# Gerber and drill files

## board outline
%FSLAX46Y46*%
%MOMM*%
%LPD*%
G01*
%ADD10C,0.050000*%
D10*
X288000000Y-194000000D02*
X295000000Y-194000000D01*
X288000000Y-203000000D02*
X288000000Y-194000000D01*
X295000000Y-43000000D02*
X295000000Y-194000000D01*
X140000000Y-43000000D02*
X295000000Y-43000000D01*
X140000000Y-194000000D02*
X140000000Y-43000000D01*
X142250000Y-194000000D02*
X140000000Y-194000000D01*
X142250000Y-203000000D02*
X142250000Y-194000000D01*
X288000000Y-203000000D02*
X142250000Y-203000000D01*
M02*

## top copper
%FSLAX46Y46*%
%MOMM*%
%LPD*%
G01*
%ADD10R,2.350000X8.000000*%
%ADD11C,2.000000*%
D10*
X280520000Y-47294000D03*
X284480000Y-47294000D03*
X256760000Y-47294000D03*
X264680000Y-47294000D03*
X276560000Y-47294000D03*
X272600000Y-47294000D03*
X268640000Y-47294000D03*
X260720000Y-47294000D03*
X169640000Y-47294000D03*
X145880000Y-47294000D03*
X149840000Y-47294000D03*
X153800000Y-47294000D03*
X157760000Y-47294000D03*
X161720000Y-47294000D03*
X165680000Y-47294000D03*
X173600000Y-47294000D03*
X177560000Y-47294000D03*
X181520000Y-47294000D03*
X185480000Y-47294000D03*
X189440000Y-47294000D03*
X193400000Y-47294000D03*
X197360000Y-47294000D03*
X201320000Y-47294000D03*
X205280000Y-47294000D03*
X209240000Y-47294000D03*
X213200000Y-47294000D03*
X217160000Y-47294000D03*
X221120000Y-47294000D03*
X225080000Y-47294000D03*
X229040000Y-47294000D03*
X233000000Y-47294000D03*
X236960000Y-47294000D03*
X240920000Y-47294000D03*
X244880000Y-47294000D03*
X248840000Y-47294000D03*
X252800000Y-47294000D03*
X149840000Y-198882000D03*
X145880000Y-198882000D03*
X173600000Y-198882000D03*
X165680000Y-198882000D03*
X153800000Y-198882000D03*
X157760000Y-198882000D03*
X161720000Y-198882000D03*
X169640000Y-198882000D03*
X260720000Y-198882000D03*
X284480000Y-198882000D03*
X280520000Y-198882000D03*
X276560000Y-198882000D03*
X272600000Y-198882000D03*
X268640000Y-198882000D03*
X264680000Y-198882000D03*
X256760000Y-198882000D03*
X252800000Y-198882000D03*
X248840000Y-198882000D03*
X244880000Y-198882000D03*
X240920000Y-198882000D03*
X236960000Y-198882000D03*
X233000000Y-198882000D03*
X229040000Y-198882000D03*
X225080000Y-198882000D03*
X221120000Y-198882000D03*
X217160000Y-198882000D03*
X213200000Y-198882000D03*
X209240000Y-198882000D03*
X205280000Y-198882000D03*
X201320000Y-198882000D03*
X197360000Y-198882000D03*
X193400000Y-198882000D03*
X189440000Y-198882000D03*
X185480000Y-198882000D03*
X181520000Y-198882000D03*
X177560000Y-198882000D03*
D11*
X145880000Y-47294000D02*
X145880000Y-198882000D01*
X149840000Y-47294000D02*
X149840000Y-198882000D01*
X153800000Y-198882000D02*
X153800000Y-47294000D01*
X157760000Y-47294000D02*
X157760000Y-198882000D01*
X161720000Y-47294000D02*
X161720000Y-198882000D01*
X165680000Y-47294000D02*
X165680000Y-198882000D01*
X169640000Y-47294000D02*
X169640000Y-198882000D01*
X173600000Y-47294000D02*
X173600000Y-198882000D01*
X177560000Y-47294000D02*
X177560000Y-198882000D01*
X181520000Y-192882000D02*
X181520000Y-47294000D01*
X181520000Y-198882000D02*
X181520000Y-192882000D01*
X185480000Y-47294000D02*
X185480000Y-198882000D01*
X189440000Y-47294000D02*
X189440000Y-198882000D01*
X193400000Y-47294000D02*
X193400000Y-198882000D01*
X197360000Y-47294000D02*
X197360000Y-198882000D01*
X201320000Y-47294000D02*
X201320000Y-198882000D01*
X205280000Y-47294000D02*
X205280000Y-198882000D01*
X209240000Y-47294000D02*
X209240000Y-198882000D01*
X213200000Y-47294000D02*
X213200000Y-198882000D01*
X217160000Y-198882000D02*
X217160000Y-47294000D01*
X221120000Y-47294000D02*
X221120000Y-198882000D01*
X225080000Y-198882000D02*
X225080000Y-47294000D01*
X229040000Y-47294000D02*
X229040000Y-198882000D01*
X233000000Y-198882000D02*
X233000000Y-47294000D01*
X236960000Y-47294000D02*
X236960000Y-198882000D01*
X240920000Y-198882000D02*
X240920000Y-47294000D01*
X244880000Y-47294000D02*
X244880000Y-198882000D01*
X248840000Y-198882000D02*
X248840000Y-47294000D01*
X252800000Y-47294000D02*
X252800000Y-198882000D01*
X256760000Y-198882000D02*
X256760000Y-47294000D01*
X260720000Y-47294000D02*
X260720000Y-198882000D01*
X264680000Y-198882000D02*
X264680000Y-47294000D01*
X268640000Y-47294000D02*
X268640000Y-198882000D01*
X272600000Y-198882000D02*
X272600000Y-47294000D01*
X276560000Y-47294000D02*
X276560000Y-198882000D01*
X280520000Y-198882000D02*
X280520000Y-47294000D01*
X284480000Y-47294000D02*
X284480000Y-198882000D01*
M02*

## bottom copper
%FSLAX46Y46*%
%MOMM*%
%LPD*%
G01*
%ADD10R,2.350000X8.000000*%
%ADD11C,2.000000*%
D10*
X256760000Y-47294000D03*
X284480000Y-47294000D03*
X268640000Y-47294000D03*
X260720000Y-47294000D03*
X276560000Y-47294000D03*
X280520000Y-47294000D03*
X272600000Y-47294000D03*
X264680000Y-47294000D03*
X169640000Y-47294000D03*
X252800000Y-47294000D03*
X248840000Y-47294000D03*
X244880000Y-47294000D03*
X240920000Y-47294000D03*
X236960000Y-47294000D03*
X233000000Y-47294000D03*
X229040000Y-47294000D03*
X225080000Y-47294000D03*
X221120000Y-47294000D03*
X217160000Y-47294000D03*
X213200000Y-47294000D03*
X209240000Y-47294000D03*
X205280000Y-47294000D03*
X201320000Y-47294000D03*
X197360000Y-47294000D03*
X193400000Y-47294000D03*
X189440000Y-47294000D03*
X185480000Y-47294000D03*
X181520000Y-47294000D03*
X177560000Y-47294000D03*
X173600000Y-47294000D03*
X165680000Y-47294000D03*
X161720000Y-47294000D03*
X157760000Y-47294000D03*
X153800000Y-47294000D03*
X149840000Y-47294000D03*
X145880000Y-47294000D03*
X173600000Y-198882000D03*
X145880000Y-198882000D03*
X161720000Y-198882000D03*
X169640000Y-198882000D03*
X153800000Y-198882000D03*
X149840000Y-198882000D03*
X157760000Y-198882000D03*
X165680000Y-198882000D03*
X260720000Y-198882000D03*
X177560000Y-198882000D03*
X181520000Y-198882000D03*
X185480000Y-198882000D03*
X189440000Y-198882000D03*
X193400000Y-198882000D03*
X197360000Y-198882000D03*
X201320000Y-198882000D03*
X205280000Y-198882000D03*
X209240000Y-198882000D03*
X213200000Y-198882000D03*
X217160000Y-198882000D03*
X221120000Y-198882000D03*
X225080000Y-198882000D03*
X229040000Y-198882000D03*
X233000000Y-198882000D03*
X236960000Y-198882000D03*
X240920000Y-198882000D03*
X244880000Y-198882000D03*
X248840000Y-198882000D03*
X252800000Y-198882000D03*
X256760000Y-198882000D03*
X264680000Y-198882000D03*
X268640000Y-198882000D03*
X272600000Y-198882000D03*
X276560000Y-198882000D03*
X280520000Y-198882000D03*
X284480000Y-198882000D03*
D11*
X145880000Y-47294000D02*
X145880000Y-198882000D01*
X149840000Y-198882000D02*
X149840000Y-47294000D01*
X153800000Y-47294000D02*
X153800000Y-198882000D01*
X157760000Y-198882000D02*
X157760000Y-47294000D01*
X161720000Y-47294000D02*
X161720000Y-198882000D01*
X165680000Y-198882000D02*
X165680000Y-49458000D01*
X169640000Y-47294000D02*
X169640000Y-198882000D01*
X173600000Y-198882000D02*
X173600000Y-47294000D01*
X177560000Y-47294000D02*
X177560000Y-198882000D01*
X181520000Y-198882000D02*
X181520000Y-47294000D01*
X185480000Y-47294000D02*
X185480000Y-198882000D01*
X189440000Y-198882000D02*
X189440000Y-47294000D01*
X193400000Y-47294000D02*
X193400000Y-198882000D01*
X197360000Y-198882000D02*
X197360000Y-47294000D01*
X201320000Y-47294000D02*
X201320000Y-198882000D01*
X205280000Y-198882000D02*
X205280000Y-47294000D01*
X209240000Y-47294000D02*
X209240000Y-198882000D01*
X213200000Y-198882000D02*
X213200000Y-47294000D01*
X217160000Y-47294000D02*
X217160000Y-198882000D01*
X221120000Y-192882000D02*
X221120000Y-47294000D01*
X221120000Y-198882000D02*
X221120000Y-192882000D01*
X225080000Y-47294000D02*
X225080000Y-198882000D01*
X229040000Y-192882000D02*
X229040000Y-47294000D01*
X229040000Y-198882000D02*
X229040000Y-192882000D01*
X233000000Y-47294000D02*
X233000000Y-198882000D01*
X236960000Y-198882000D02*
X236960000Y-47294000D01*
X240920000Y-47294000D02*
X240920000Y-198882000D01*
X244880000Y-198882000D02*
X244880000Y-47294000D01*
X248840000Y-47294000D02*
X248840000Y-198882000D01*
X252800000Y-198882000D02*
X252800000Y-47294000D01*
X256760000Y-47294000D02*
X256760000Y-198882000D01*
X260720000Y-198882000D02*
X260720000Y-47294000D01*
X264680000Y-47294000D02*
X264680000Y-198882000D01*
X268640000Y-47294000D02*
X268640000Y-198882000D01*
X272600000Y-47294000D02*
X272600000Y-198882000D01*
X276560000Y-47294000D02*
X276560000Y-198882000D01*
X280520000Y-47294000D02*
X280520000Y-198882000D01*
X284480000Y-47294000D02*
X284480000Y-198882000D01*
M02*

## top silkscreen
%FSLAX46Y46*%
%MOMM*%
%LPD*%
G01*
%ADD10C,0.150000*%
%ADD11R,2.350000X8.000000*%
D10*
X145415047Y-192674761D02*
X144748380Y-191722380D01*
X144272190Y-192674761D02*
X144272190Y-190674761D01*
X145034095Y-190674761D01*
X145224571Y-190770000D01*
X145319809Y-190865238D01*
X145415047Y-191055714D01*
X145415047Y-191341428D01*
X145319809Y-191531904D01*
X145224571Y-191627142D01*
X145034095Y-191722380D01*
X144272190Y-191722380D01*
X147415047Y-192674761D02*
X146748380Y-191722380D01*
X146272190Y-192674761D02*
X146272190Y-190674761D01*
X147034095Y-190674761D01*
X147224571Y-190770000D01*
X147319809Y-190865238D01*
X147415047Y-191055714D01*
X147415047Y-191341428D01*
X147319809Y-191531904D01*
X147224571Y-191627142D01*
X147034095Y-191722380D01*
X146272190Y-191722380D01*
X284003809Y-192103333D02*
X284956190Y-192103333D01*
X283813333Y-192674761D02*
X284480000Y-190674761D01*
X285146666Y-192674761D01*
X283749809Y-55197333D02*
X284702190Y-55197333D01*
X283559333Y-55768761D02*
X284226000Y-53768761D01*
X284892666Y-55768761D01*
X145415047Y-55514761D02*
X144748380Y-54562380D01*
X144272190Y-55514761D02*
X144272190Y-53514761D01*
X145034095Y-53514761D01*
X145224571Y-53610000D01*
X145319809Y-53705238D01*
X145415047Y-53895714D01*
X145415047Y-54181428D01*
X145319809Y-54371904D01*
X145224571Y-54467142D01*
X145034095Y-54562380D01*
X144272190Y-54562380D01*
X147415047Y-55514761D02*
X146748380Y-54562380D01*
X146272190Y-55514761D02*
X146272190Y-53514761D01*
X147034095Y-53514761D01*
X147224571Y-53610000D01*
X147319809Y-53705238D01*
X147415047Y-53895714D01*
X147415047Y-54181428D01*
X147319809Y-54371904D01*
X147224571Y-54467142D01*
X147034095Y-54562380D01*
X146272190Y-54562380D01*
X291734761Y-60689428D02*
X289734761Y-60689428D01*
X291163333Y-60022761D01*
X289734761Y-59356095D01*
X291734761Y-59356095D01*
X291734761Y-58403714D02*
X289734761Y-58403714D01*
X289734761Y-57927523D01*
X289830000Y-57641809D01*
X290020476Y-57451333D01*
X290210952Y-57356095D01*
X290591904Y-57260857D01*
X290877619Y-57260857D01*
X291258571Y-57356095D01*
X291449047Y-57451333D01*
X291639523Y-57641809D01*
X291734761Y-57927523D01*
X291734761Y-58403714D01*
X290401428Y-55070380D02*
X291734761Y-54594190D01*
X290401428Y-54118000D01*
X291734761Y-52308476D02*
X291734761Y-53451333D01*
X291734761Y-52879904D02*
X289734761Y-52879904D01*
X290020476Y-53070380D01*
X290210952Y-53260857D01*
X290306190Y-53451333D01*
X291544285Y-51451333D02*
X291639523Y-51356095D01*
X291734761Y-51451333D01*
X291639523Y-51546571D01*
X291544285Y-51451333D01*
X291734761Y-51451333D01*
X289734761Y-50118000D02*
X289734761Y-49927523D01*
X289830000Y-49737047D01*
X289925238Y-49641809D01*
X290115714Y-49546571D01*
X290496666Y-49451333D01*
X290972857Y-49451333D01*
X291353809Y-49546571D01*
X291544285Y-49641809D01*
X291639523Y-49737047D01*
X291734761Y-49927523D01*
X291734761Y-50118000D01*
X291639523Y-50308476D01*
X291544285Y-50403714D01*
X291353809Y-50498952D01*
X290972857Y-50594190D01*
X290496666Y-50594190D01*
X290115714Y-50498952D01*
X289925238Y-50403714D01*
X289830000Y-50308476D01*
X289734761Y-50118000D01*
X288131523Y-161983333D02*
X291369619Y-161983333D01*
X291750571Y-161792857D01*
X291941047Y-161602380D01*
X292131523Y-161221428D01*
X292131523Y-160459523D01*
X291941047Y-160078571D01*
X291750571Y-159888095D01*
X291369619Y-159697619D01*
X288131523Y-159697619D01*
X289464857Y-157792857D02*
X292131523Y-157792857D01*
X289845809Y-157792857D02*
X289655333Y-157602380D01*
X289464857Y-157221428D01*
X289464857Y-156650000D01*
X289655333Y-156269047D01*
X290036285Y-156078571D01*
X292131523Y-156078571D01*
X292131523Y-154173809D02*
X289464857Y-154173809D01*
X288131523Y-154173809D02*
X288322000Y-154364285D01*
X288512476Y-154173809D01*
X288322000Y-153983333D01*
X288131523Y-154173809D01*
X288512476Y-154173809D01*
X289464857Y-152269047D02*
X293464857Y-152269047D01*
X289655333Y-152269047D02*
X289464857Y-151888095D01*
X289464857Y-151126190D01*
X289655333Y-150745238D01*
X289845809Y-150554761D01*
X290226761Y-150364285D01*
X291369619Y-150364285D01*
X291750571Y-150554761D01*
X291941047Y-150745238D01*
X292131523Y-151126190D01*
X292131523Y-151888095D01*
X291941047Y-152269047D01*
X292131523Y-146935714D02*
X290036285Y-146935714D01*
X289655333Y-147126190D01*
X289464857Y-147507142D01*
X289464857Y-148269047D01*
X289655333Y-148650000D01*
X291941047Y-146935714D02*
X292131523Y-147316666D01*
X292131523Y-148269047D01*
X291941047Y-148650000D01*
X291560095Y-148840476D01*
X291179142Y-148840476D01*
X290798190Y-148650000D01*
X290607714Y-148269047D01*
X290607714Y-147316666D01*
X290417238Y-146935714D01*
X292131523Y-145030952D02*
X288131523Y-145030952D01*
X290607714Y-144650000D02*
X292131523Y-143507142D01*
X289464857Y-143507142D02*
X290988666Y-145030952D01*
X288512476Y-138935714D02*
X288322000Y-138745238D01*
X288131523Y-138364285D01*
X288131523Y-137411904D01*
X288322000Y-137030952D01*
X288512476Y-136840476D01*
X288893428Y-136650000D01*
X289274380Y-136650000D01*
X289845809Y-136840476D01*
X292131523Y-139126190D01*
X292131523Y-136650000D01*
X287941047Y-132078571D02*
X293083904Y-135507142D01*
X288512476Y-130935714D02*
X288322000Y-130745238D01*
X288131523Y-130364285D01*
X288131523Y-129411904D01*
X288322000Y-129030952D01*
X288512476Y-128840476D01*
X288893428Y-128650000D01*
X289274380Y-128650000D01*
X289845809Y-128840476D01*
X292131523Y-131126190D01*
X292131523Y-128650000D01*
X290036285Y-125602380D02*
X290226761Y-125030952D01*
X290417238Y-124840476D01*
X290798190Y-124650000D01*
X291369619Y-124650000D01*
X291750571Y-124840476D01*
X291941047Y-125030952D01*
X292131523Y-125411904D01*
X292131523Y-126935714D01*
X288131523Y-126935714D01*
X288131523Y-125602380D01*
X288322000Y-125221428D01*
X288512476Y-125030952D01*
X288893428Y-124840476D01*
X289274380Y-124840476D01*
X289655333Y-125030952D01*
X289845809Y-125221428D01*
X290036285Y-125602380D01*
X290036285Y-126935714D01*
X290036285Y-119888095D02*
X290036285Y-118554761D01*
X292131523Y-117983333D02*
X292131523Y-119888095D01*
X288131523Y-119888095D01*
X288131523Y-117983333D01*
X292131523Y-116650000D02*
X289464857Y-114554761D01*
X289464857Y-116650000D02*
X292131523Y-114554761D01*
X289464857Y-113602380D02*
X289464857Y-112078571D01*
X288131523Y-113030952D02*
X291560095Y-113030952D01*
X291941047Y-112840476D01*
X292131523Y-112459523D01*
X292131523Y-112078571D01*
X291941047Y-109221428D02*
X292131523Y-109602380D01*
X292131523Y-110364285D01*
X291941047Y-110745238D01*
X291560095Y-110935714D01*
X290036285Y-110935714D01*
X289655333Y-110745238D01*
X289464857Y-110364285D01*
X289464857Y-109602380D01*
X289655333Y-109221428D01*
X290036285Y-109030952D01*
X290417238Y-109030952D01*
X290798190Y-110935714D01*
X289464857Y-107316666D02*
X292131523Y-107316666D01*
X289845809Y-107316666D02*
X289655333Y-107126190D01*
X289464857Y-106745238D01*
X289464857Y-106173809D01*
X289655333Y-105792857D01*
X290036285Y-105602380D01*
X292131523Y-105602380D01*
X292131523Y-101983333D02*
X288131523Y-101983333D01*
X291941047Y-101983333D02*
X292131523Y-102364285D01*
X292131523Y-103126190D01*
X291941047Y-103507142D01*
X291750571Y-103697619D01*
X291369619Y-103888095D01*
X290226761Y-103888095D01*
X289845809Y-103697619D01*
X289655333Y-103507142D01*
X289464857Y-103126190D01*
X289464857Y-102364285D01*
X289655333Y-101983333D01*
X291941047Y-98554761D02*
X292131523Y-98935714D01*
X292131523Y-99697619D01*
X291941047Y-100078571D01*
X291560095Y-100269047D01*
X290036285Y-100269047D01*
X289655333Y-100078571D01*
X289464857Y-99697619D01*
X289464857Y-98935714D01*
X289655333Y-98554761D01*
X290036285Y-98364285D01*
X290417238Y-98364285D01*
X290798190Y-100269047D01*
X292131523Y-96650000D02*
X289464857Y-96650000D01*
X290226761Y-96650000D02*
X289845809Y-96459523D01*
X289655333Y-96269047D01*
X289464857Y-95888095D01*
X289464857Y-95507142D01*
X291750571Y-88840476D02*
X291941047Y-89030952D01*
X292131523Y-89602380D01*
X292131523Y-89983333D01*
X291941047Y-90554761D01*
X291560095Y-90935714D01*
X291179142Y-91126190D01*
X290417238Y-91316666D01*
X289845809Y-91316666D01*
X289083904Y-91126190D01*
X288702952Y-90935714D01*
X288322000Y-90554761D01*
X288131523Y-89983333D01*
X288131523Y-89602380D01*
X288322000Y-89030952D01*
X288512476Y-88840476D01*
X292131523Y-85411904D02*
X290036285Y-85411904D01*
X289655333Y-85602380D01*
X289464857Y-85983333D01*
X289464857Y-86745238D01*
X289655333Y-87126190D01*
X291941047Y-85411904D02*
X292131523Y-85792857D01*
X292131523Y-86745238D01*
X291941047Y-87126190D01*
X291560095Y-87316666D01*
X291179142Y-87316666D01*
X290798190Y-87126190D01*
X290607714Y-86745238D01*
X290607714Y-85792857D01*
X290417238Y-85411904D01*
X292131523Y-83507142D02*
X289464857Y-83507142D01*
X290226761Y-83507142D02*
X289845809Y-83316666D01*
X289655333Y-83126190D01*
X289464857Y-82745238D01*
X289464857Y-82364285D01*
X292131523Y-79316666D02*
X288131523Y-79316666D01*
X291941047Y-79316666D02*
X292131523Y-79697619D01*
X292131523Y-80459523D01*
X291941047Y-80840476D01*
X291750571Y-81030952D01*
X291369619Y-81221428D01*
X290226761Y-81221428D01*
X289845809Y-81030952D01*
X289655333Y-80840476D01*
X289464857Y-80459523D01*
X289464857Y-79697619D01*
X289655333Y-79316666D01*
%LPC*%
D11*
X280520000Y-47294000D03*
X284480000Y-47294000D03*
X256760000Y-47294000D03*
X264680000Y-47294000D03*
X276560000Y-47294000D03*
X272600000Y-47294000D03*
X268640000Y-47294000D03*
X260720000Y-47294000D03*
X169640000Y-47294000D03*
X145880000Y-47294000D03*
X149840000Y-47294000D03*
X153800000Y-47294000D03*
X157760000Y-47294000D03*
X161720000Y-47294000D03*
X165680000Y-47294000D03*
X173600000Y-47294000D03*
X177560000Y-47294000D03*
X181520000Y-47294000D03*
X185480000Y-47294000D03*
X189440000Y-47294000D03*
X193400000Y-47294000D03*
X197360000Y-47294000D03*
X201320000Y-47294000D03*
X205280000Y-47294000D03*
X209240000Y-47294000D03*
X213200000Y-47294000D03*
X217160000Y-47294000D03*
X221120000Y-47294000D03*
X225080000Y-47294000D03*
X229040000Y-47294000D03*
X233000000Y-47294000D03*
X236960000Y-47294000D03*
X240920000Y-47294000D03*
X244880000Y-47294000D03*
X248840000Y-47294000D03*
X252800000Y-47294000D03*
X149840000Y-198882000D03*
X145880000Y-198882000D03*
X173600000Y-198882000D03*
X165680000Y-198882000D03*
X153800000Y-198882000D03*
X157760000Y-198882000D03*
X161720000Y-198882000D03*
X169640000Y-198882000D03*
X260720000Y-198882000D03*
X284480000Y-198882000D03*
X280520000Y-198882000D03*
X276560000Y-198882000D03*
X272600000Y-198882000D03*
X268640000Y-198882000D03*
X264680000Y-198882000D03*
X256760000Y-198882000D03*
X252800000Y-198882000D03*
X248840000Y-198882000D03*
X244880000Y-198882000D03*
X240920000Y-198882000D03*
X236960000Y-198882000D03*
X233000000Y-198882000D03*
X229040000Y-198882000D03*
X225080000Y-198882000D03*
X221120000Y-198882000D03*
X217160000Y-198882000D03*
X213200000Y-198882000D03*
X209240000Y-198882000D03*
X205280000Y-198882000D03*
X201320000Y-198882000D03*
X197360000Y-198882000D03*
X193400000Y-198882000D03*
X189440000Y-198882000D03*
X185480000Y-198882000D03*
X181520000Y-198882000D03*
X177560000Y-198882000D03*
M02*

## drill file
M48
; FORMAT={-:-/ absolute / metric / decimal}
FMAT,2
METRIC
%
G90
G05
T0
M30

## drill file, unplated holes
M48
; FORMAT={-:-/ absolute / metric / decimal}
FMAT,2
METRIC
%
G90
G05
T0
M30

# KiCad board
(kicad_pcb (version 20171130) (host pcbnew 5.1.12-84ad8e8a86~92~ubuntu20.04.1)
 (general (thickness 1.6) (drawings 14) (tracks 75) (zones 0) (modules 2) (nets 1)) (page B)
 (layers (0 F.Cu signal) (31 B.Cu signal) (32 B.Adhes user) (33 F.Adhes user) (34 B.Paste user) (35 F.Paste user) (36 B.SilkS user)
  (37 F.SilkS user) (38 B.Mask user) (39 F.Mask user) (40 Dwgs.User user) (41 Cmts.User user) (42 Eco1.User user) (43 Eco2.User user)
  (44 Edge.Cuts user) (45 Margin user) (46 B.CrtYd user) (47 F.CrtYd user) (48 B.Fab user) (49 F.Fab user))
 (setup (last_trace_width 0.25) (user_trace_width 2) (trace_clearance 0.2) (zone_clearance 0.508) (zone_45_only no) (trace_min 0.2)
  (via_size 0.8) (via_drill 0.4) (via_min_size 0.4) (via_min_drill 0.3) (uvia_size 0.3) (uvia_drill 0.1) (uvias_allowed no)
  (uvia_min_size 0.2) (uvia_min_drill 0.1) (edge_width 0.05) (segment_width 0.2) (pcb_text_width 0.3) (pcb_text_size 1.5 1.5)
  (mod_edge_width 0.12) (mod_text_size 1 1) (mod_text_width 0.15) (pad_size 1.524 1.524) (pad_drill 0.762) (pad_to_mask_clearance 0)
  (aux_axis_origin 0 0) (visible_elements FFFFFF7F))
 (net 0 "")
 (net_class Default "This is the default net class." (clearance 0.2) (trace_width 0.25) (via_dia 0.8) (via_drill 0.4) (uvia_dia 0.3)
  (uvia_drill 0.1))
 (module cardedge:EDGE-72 (layer F.Cu) (at 200.34 66.294)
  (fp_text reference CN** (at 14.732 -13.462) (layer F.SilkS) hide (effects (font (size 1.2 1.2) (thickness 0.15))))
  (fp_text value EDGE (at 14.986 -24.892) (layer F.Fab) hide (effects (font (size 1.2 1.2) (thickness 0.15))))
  (pad PP smd rect (at 80.18 -19) (size 2.35 8) (layers F.Cu F.Paste F.Mask))
  (pad RR smd rect (at 84.14 -19) (size 2.35 8) (layers F.Cu F.Paste F.Mask))
  (pad 29 smd rect (at 56.42 -19) (size 2.35 8) (layers B.Cu B.Paste B.Mask))
  (pad 36 smd rect (at 84.14 -19) (size 2.35 8) (layers B.Cu B.Paste B.Mask))
  (pad 32 smd rect (at 68.3 -19) (size 2.35 8) (layers B.Cu B.Paste B.Mask))
  (pad 30 smd rect (at 60.38 -19) (size 2.35 8) (layers B.Cu B.Paste B.Mask))
  (pad 34 smd rect (at 76.22 -19) (size 2.35 8) (layers B.Cu B.Paste B.Mask))
  (pad 35 smd rect (at 80.18 -19) (size 2.35 8) (layers B.Cu B.Paste B.Mask))
  (pad 33 smd rect (at 72.26 -19) (size 2.35 8) (layers B.Cu B.Paste B.Mask))
  (pad HH smd rect (at 56.42 -19) (size 2.35 8) (layers F.Cu F.Paste F.Mask))
  (pad KK smd rect (at 64.34 -19) (size 2.35 8) (layers F.Cu F.Paste F.Mask))
  (pad NN smd rect (at 76.22 -19) (size 2.35 8) (layers F.Cu F.Paste F.Mask))
  (pad MM smd rect (at 72.26 -19) (size 2.35 8) (layers F.Cu F.Paste F.Mask))
  (pad LL smd rect (at 68.3 -19) (size 2.35 8) (layers F.Cu F.Paste F.Mask))
  (pad 31 smd rect (at 64.34 -19) (size 2.35 8) (layers B.Cu B.Paste B.Mask))
  (pad JJ smd rect (at 60.38 -19) (size 2.35 8) (layers F.Cu F.Paste F.Mask))
  (pad H smd rect (at -30.7 -19) (size 2.35 8) (layers F.Cu F.Paste F.Mask))
  (pad 7 smd rect (at -30.7 -19) (size 2.35 8) (layers B.Cu B.Paste B.Mask))
  (pad 28 smd rect (at 52.46 -19) (size 2.35 8) (layers B.Cu B.Paste B.Mask))
  (pad 27 smd rect (at 48.5 -19) (size 2.35 8) (layers B.Cu B.Paste B.Mask))
  (pad 26 smd rect (at 44.54 -19) (size 2.35 8) (layers B.Cu B.Paste B.Mask))
  (pad 25 smd rect (at 40.58 -19) (size 2.35 8) (layers B.Cu B.Paste B.Mask))
  (pad 24 smd rect (at 36.62 -19) (size 2.35 8) (layers B.Cu B.Paste B.Mask))
  (pad 23 smd rect (at 32.66 -19) (size 2.35 8) (layers B.Cu B.Paste B.Mask))
  (pad 22 smd rect (at 28.7 -19) (size 2.35 8) (layers B.Cu B.Paste B.Mask))
  (pad 21 smd rect (at 24.74 -19) (size 2.35 8) (layers B.Cu B.Paste B.Mask))
  (pad 20 smd rect (at 20.78 -19) (size 2.35 8) (layers B.Cu B.Paste B.Mask))
  (pad 19 smd rect (at 16.82 -19) (size 2.35 8) (layers B.Cu B.Paste B.Mask))
  (pad 18 smd rect (at 12.86 -19) (size 2.35 8) (layers B.Cu B.Paste B.Mask))
  (pad 17 smd rect (at 8.9 -19) (size 2.35 8) (layers B.Cu B.Paste B.Mask))
  (pad 16 smd rect (at 4.94 -19) (size 2.35 8) (layers B.Cu B.Paste B.Mask))
  (pad 15 smd rect (at 0.98 -19) (size 2.35 8) (layers B.Cu B.Paste B.Mask))
  (pad 14 smd rect (at -2.98 -19) (size 2.35 8) (layers B.Cu B.Paste B.Mask))
  (pad 13 smd rect (at -6.94 -19) (size 2.35 8) (layers B.Cu B.Paste B.Mask))
  (pad 12 smd rect (at -10.9 -19) (size 2.35 8) (layers B.Cu B.Paste B.Mask))
  (pad 11 smd rect (at -14.86 -19) (size 2.35 8) (layers B.Cu B.Paste B.Mask))
  (pad 10 smd rect (at -18.82 -19) (size 2.35 8) (layers B.Cu B.Paste B.Mask))
  (pad 9 smd rect (at -22.78 -19) (size 2.35 8) (layers B.Cu B.Paste B.Mask))
  (pad 8 smd rect (at -26.74 -19) (size 2.35 8) (layers B.Cu B.Paste B.Mask))
  (pad 6 smd rect (at -34.66 -19) (size 2.35 8) (layers B.Cu B.Paste B.Mask))
  (pad 5 smd rect (at -38.62 -19) (size 2.35 8) (layers B.Cu B.Paste B.Mask))
  (pad 4 smd rect (at -42.58 -19) (size 2.35 8) (layers B.Cu B.Paste B.Mask))
  (pad 3 smd rect (at -46.54 -19) (size 2.35 8) (layers B.Cu B.Paste B.Mask))
  (pad 2 smd rect (at -50.5 -19) (size 2.35 8) (layers B.Cu B.Paste B.Mask))
  (pad 1 smd rect (at -54.46 -19) (size 2.35 8) (layers B.Cu B.Paste B.Mask))
  (pad A smd rect (at -54.46 -19) (size 2.35 8) (layers F.Cu F.Paste F.Mask))
  (pad B smd rect (at -50.5 -19) (size 2.35 8) (layers F.Cu F.Paste F.Mask))
  (pad C smd rect (at -46.54 -19) (size 2.35 8) (layers F.Cu F.Paste F.Mask))
  (pad D smd rect (at -42.58 -19) (size 2.35 8) (layers F.Cu F.Paste F.Mask))
  (pad E smd rect (at -38.62 -19) (size 2.35 8) (layers F.Cu F.Paste F.Mask))
  (pad F smd rect (at -34.66 -19) (size 2.35 8) (layers F.Cu F.Paste F.Mask))
  (pad J smd rect (at -26.74 -19) (size 2.35 8) (layers F.Cu F.Paste F.Mask))
  (pad K smd rect (at -22.78 -19) (size 2.35 8) (layers F.Cu F.Paste F.Mask))
  (pad L smd rect (at -18.82 -19) (size 2.35 8) (layers F.Cu F.Paste F.Mask))
  (pad M smd rect (at -14.86 -19) (size 2.35 8) (layers F.Cu F.Paste F.Mask))
  (pad N smd rect (at -10.9 -19) (size 2.35 8) (layers F.Cu F.Paste F.Mask))
  (pad P smd rect (at -6.94 -19) (size 2.35 8) (layers F.Cu F.Paste F.Mask))
  (pad R smd rect (at -2.98 -19) (size 2.35 8) (layers F.Cu F.Paste F.Mask))
  (pad S smd rect (at 0.98 -19) (size 2.35 8) (layers F.Cu F.Paste F.Mask))
  (pad T smd rect (at 4.94 -19) (size 2.35 8) (layers F.Cu F.Paste F.Mask))
  (pad U smd rect (at 8.9 -19) (size 2.35 8) (layers F.Cu F.Paste F.Mask))
  (pad V smd rect (at 12.86 -19) (size 2.35 8) (layers F.Cu F.Paste F.Mask))
  (pad W smd rect (at 16.82 -19) (size 2.35 8) (layers F.Cu F.Paste F.Mask))
  (pad X smd rect (at 20.78 -19) (size 2.35 8) (layers F.Cu F.Paste F.Mask))
  (pad Y smd rect (at 24.74 -19) (size 2.35 8) (layers F.Cu F.Paste F.Mask))
  (pad Z smd rect (at 28.7 -19) (size 2.35 8) (layers F.Cu F.Paste F.Mask))
  (pad AA smd rect (at 32.66 -19) (size 2.35 8) (layers F.Cu F.Paste F.Mask))
  (pad BB smd rect (at 36.62 -19) (size 2.35 8) (layers F.Cu F.Paste F.Mask))
  (pad CC smd rect (at 40.58 -19) (size 2.35 8) (layers F.Cu F.Paste F.Mask))
  (pad DD smd rect (at 44.54 -19) (size 2.35 8) (layers F.Cu F.Paste F.Mask))
  (pad EE smd rect (at 48.5 -19) (size 2.35 8) (layers F.Cu F.Paste F.Mask))
  (pad FF smd rect (at 52.46 -19) (size 2.35 8) (layers F.Cu F.Paste F.Mask)))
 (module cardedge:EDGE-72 (layer F.Cu) (at 230.02 179.882 180)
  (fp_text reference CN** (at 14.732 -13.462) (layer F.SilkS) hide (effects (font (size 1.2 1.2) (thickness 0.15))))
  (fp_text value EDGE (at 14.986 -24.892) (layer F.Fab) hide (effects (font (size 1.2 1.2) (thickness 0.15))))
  (pad PP smd rect (at 80.18 -19 180) (size 2.35 8) (layers F.Cu F.Paste F.Mask))
  (pad RR smd rect (at 84.14 -19 180) (size 2.35 8) (layers F.Cu F.Paste F.Mask))
  (pad 29 smd rect (at 56.42 -19 180) (size 2.35 8) (layers B.Cu B.Paste B.Mask))
  (pad 36 smd rect (at 84.14 -19 180) (size 2.35 8) (layers B.Cu B.Paste B.Mask))
  (pad 32 smd rect (at 68.3 -19 180) (size 2.35 8) (layers B.Cu B.Paste B.Mask))
  (pad 30 smd rect (at 60.38 -19 180) (size 2.35 8) (layers B.Cu B.Paste B.Mask))
  (pad 34 smd rect (at 76.22 -19 180) (size 2.35 8) (layers B.Cu B.Paste B.Mask))
  (pad 35 smd rect (at 80.18 -19 180) (size 2.35 8) (layers B.Cu B.Paste B.Mask))
  (pad 33 smd rect (at 72.26 -19 180) (size 2.35 8) (layers B.Cu B.Paste B.Mask))
  (pad HH smd rect (at 56.42 -19 180) (size 2.35 8) (layers F.Cu F.Paste F.Mask))
  (pad KK smd rect (at 64.34 -19 180) (size 2.35 8) (layers F.Cu F.Paste F.Mask))
  (pad NN smd rect (at 76.22 -19 180) (size 2.35 8) (layers F.Cu F.Paste F.Mask))
  (pad MM smd rect (at 72.26 -19 180) (size 2.35 8) (layers F.Cu F.Paste F.Mask))
  (pad LL smd rect (at 68.3 -19 180) (size 2.35 8) (layers F.Cu F.Paste F.Mask))
  (pad 31 smd rect (at 64.34 -19 180) (size 2.35 8) (layers B.Cu B.Paste B.Mask))
  (pad JJ smd rect (at 60.38 -19 180) (size 2.35 8) (layers F.Cu F.Paste F.Mask))
  (pad H smd rect (at -30.7 -19 180) (size 2.35 8) (layers F.Cu F.Paste F.Mask))
  (pad 7 smd rect (at -30.7 -19 180) (size 2.35 8) (layers B.Cu B.Paste B.Mask))
  (pad 28 smd rect (at 52.46 -19 180) (size 2.35 8) (layers B.Cu B.Paste B.Mask))
  (pad 27 smd rect (at 48.5 -19 180) (size 2.35 8) (layers B.Cu B.Paste B.Mask))
  (pad 26 smd rect (at 44.54 -19 180) (size 2.35 8) (layers B.Cu B.Paste B.Mask))
  (pad 25 smd rect (at 40.58 -19 180) (size 2.35 8) (layers B.Cu B.Paste B.Mask))
  (pad 24 smd rect (at 36.62 -19 180) (size 2.35 8) (layers B.Cu B.Paste B.Mask))
  (pad 23 smd rect (at 32.66 -19 180) (size 2.35 8) (layers B.Cu B.Paste B.Mask))
  (pad 22 smd rect (at 28.7 -19 180) (size 2.35 8) (layers B.Cu B.Paste B.Mask))
  (pad 21 smd rect (at 24.74 -19 180) (size 2.35 8) (layers B.Cu B.Paste B.Mask))
  (pad 20 smd rect (at 20.78 -19 180) (size 2.35 8) (layers B.Cu B.Paste B.Mask))
  (pad 19 smd rect (at 16.82 -19 180) (size 2.35 8) (layers B.Cu B.Paste B.Mask))
  (pad 18 smd rect (at 12.86 -19 180) (size 2.35 8) (layers B.Cu B.Paste B.Mask))
  (pad 17 smd rect (at 8.9 -19 180) (size 2.35 8) (layers B.Cu B.Paste B.Mask))
  (pad 16 smd rect (at 4.94 -19 180) (size 2.35 8) (layers B.Cu B.Paste B.Mask))
  (pad 15 smd rect (at 0.98 -19 180) (size 2.35 8) (layers B.Cu B.Paste B.Mask))
  (pad 14 smd rect (at -2.98 -19 180) (size 2.35 8) (layers B.Cu B.Paste B.Mask))
  (pad 13 smd rect (at -6.94 -19 180) (size 2.35 8) (layers B.Cu B.Paste B.Mask))
  (pad 12 smd rect (at -10.9 -19 180) (size 2.35 8) (layers B.Cu B.Paste B.Mask))
  (pad 11 smd rect (at -14.86 -19 180) (size 2.35 8) (layers B.Cu B.Paste B.Mask))
  (pad 10 smd rect (at -18.82 -19 180) (size 2.35 8) (layers B.Cu B.Paste B.Mask))
  (pad 9 smd rect (at -22.78 -19 180) (size 2.35 8) (layers B.Cu B.Paste B.Mask))
  (pad 8 smd rect (at -26.74 -19 180) (size 2.35 8) (layers B.Cu B.Paste B.Mask))
  (pad 6 smd rect (at -34.66 -19 180) (size 2.35 8) (layers B.Cu B.Paste B.Mask))
  (pad 5 smd rect (at -38.62 -19 180) (size 2.35 8) (layers B.Cu B.Paste B.Mask))
  (pad 4 smd rect (at -42.58 -19 180) (size 2.35 8) (layers B.Cu B.Paste B.Mask))
  (pad 3 smd rect (at -46.54 -19 180) (size 2.35 8) (layers B.Cu B.Paste B.Mask))
  (pad 2 smd rect (at -50.5 -19 180) (size 2.35 8) (layers B.Cu B.Paste B.Mask))
  (pad 1 smd rect (at -54.46 -19 180) (size 2.35 8) (layers B.Cu B.Paste B.Mask))
  (pad A smd rect (at -54.46 -19 180) (size 2.35 8) (layers F.Cu F.Paste F.Mask))
  (pad B smd rect (at -50.5 -19 180) (size 2.35 8) (layers F.Cu F.Paste F.Mask))
  (pad C smd rect (at -46.54 -19 180) (size 2.35 8) (layers F.Cu F.Paste F.Mask))
  (pad D smd rect (at -42.58 -19 180) (size 2.35 8) (layers F.Cu F.Paste F.Mask))
  (pad E smd rect (at -38.62 -19 180) (size 2.35 8) (layers F.Cu F.Paste F.Mask))
  (pad F smd rect (at -34.66 -19 180) (size 2.35 8) (layers F.Cu F.Paste F.Mask))
  (pad J smd rect (at -26.74 -19 180) (size 2.35 8) (layers F.Cu F.Paste F.Mask))
  (pad K smd rect (at -22.78 -19 180) (size 2.35 8) (layers F.Cu F.Paste F.Mask))
  (pad L smd rect (at -18.82 -19 180) (size 2.35 8) (layers F.Cu F.Paste F.Mask))
  (pad M smd rect (at -14.86 -19 180) (size 2.35 8) (layers F.Cu F.Paste F.Mask))
  (pad N smd rect (at -10.9 -19 180) (size 2.35 8) (layers F.Cu F.Paste F.Mask))
  (pad P smd rect (at -6.94 -19 180) (size 2.35 8) (layers F.Cu F.Paste F.Mask))
  (pad R smd rect (at -2.98 -19 180) (size 2.35 8) (layers F.Cu F.Paste F.Mask))
  (pad S smd rect (at 0.98 -19 180) (size 2.35 8) (layers F.Cu F.Paste F.Mask))
  (pad T smd rect (at 4.94 -19 180) (size 2.35 8) (layers F.Cu F.Paste F.Mask))
  (pad U smd rect (at 8.9 -19 180) (size 2.35 8) (layers F.Cu F.Paste F.Mask))
  (pad V smd rect (at 12.86 -19 180) (size 2.35 8) (layers F.Cu F.Paste F.Mask))
  (pad W smd rect (at 16.82 -19 180) (size 2.35 8) (layers F.Cu F.Paste F.Mask))
  (pad X smd rect (at 20.78 -19 180) (size 2.35 8) (layers F.Cu F.Paste F.Mask))
  (pad Y smd rect (at 24.74 -19 180) (size 2.35 8) (layers F.Cu F.Paste F.Mask))
  (pad Z smd rect (at 28.7 -19 180) (size 2.35 8) (layers F.Cu F.Paste F.Mask))
  (pad AA smd rect (at 32.66 -19 180) (size 2.35 8) (layers F.Cu F.Paste F.Mask))
  (pad BB smd rect (at 36.62 -19 180) (size 2.35 8) (layers F.Cu F.Paste F.Mask))
  (pad CC smd rect (at 40.58 -19 180) (size 2.35 8) (layers F.Cu F.Paste F.Mask))
  (pad DD smd rect (at 44.54 -19 180) (size 2.35 8) (layers F.Cu F.Paste F.Mask))
  (pad EE smd rect (at 48.5 -19 180) (size 2.35 8) (layers F.Cu F.Paste F.Mask))
  (pad FF smd rect (at 52.46 -19 180) (size 2.35 8) (layers F.Cu F.Paste F.Mask)))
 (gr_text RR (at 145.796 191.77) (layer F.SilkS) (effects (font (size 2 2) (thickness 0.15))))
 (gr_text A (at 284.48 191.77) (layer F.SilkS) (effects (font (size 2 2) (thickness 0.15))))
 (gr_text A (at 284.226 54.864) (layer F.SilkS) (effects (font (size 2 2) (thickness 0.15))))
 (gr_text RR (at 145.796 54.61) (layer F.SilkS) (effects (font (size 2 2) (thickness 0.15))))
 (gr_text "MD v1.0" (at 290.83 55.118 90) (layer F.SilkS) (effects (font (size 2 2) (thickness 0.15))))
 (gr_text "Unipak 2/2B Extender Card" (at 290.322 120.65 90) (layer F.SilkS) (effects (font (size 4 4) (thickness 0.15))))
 (gr_line (start 288 194) (end 295 194) (layer Edge.Cuts) (width 0.05))
 (gr_line (start 288 203) (end 288 194) (layer Edge.Cuts) (width 0.05))
 (gr_line (start 295 43) (end 295 194) (layer Edge.Cuts) (width 0.05))
 (gr_line (start 140 43) (end 295 43) (layer Edge.Cuts) (width 0.05))
 (gr_line (start 140 194) (end 140 43) (layer Edge.Cuts) (width 0.05))
 (gr_line (start 142.25 194) (end 140 194) (layer Edge.Cuts) (width 0.05))
 (gr_line (start 142.25 203) (end 142.25 194) (layer Edge.Cuts) (width 0.05))
 (gr_line (start 288 203) (end 142.25 203) (layer Edge.Cuts) (width 0.05))
 (segment (start 145.88 47.294) (end 145.88 198.882) (width 2) (layer F.Cu) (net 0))
 (segment (start 149.84 47.294) (end 149.84 198.882) (width 2) (layer F.Cu) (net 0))
 (segment (start 153.8 198.882) (end 153.8 47.294) (width 2) (layer F.Cu) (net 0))
 (segment (start 157.76 47.294) (end 157.76 198.882) (width 2) (layer F.Cu) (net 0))
 (segment (start 161.72 47.294) (end 161.72 198.882) (width 2) (layer F.Cu) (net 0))
 (segment (start 165.68 47.294) (end 165.68 198.882) (width 2) (layer F.Cu) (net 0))
 (segment (start 169.64 47.294) (end 169.64 198.882) (width 2) (layer F.Cu) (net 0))
 (segment (start 173.6 47.294) (end 173.6 198.882) (width 2) (layer F.Cu) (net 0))
 (segment (start 177.56 47.294) (end 177.56 198.882) (width 2) (layer F.Cu) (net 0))
 (segment (start 181.52 192.882) (end 181.52 47.294) (width 2) (layer F.Cu) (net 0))
 (segment (start 181.52 198.882) (end 181.52 192.882) (width 2) (layer F.Cu) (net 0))
 (segment (start 185.48 47.294) (end 185.48 198.882) (width 2) (layer F.Cu) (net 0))
 (segment (start 189.44 47.294) (end 189.44 198.882) (width 2) (layer F.Cu) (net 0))
 (segment (start 193.4 47.294) (end 193.4 198.882) (width 2) (layer F.Cu) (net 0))
 (segment (start 197.36 47.294) (end 197.36 198.882) (width 2) (layer F.Cu) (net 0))
 (segment (start 201.32 47.294) (end 201.32 198.882) (width 2) (layer F.Cu) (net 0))
 (segment (start 205.28 47.294) (end 205.28 198.882) (width 2) (layer F.Cu) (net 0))
 (segment (start 209.24 47.294) (end 209.24 198.882) (width 2) (layer F.Cu) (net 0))
 (segment (start 213.2 47.294) (end 213.2 198.882) (width 2) (layer F.Cu) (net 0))
 (segment (start 217.16 198.882) (end 217.16 47.294) (width 2) (layer F.Cu) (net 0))
 (segment (start 221.12 47.294) (end 221.12 198.882) (width 2) (layer F.Cu) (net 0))
 (segment (start 225.08 198.882) (end 225.08 47.294) (width 2) (layer F.Cu) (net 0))
 (segment (start 229.04 47.294) (end 229.04 198.882) (width 2) (layer F.Cu) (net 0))
 (segment (start 233 198.882) (end 233 47.294) (width 2) (layer F.Cu) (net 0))
 (segment (start 236.96 47.294) (end 236.96 198.882) (width 2) (layer F.Cu) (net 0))
 (segment (start 240.92 198.882) (end 240.92 47.294) (width 2) (layer F.Cu) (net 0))
 (segment (start 244.88 47.294) (end 244.88 198.882) (width 2) (layer F.Cu) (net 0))
 (segment (start 248.84 198.882) (end 248.84 47.294) (width 2) (layer F.Cu) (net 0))
 (segment (start 252.8 47.294) (end 252.8 198.882) (width 2) (layer F.Cu) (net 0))
 (segment (start 256.76 198.882) (end 256.76 47.294) (width 2) (layer F.Cu) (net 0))
 (segment (start 260.72 47.294) (end 260.72 198.882) (width 2) (layer F.Cu) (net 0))
 (segment (start 264.68 198.882) (end 264.68 47.294) (width 2) (layer F.Cu) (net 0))
 (segment (start 268.64 47.294) (end 268.64 198.882) (width 2) (layer F.Cu) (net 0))
 (segment (start 272.6 198.882) (end 272.6 47.294) (width 2) (layer F.Cu) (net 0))
 (segment (start 276.56 47.294) (end 276.56 198.882) (width 2) (layer F.Cu) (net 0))
 (segment (start 280.52 198.882) (end 280.52 47.294) (width 2) (layer F.Cu) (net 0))
 (segment (start 284.48 47.294) (end 284.48 198.882) (width 2) (layer F.Cu) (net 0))
 (segment (start 145.88 47.294) (end 145.88 198.882) (width 2) (layer B.Cu) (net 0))
 (segment (start 149.84 198.882) (end 149.84 47.294) (width 2) (layer B.Cu) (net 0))
 (segment (start 153.8 47.294) (end 153.8 198.882) (width 2) (layer B.Cu) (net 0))
 (segment (start 157.76 198.882) (end 157.76 47.294) (width 2) (layer B.Cu) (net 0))
 (segment (start 161.72 47.294) (end 161.72 198.882) (width 2) (layer B.Cu) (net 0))
 (segment (start 165.68 198.882) (end 165.68 49.458) (width 2) (layer B.Cu) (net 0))
 (segment (start 169.64 47.294) (end 169.64 198.882) (width 2) (layer B.Cu) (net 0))
 (segment (start 173.6 198.882) (end 173.6 47.294) (width 2) (layer B.Cu) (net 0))
 (segment (start 177.56 47.294) (end 177.56 198.882) (width 2) (layer B.Cu) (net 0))
 (segment (start 181.52 198.882) (end 181.52 47.294) (width 2) (layer B.Cu) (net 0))
 (segment (start 185.48 47.294) (end 185.48 198.882) (width 2) (layer B.Cu) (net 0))
 (segment (start 189.44 198.882) (end 189.44 47.294) (width 2) (layer B.Cu) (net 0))
 (segment (start 193.4 47.294) (end 193.4 198.882) (width 2) (layer B.Cu) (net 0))
 (segment (start 197.36 198.882) (end 197.36 47.294) (width 2) (layer B.Cu) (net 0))
 (segment (start 201.32 47.294) (end 201.32 198.882) (width 2) (layer B.Cu) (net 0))
 (segment (start 205.28 198.882) (end 205.28 47.294) (width 2) (layer B.Cu) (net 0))
 (segment (start 209.24 47.294) (end 209.24 198.882) (width 2) (layer B.Cu) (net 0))
 (segment (start 213.2 198.882) (end 213.2 47.294) (width 2) (layer B.Cu) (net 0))
 (segment (start 217.16 47.294) (end 217.16 198.882) (width 2) (layer B.Cu) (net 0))
 (segment (start 221.12 192.882) (end 221.12 47.294) (width 2) (layer B.Cu) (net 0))
 (segment (start 221.12 198.882) (end 221.12 192.882) (width 2) (layer B.Cu) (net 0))
 (segment (start 225.08 47.294) (end 225.08 198.882) (width 2) (layer B.Cu) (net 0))
 (segment (start 229.04 192.882) (end 229.04 47.294) (width 2) (layer B.Cu) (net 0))
 (segment (start 229.04 198.882) (end 229.04 192.882) (width 2) (layer B.Cu) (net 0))
 (segment (start 233 47.294) (end 233 198.882) (width 2) (layer B.Cu) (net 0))
 (segment (start 236.96 198.882) (end 236.96 47.294) (width 2) (layer B.Cu) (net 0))
 (segment (start 240.92 47.294) (end 240.92 198.882) (width 2) (layer B.Cu) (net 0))
 (segment (start 244.88 198.882) (end 244.88 47.294) (width 2) (layer B.Cu) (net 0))
 (segment (start 248.84 47.294) (end 248.84 198.882) (width 2) (layer B.Cu) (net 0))
 (segment (start 252.8 198.882) (end 252.8 47.294) (width 2) (layer B.Cu) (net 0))
 (segment (start 256.76 47.294) (end 256.76 198.882) (width 2) (layer B.Cu) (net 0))
 (segment (start 260.72 198.882) (end 260.72 47.294) (width 2) (layer B.Cu) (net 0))
 (segment (start 264.68 47.294) (end 264.68 198.882) (width 2) (layer B.Cu) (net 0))
 (segment (start 268.64 47.294) (end 268.64 198.882) (width 2) (layer B.Cu) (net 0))
 (segment (start 272.6 47.294) (end 272.6 198.882) (width 2) (layer B.Cu) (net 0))
 (segment (start 276.56 47.294) (end 276.56 198.882) (width 2) (layer B.Cu) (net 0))
 (segment (start 280.52 47.294) (end 280.52 198.882) (width 2) (layer B.Cu) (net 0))
 (segment (start 284.48 47.294) (end 284.48 198.882) (width 2) (layer B.Cu) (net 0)))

